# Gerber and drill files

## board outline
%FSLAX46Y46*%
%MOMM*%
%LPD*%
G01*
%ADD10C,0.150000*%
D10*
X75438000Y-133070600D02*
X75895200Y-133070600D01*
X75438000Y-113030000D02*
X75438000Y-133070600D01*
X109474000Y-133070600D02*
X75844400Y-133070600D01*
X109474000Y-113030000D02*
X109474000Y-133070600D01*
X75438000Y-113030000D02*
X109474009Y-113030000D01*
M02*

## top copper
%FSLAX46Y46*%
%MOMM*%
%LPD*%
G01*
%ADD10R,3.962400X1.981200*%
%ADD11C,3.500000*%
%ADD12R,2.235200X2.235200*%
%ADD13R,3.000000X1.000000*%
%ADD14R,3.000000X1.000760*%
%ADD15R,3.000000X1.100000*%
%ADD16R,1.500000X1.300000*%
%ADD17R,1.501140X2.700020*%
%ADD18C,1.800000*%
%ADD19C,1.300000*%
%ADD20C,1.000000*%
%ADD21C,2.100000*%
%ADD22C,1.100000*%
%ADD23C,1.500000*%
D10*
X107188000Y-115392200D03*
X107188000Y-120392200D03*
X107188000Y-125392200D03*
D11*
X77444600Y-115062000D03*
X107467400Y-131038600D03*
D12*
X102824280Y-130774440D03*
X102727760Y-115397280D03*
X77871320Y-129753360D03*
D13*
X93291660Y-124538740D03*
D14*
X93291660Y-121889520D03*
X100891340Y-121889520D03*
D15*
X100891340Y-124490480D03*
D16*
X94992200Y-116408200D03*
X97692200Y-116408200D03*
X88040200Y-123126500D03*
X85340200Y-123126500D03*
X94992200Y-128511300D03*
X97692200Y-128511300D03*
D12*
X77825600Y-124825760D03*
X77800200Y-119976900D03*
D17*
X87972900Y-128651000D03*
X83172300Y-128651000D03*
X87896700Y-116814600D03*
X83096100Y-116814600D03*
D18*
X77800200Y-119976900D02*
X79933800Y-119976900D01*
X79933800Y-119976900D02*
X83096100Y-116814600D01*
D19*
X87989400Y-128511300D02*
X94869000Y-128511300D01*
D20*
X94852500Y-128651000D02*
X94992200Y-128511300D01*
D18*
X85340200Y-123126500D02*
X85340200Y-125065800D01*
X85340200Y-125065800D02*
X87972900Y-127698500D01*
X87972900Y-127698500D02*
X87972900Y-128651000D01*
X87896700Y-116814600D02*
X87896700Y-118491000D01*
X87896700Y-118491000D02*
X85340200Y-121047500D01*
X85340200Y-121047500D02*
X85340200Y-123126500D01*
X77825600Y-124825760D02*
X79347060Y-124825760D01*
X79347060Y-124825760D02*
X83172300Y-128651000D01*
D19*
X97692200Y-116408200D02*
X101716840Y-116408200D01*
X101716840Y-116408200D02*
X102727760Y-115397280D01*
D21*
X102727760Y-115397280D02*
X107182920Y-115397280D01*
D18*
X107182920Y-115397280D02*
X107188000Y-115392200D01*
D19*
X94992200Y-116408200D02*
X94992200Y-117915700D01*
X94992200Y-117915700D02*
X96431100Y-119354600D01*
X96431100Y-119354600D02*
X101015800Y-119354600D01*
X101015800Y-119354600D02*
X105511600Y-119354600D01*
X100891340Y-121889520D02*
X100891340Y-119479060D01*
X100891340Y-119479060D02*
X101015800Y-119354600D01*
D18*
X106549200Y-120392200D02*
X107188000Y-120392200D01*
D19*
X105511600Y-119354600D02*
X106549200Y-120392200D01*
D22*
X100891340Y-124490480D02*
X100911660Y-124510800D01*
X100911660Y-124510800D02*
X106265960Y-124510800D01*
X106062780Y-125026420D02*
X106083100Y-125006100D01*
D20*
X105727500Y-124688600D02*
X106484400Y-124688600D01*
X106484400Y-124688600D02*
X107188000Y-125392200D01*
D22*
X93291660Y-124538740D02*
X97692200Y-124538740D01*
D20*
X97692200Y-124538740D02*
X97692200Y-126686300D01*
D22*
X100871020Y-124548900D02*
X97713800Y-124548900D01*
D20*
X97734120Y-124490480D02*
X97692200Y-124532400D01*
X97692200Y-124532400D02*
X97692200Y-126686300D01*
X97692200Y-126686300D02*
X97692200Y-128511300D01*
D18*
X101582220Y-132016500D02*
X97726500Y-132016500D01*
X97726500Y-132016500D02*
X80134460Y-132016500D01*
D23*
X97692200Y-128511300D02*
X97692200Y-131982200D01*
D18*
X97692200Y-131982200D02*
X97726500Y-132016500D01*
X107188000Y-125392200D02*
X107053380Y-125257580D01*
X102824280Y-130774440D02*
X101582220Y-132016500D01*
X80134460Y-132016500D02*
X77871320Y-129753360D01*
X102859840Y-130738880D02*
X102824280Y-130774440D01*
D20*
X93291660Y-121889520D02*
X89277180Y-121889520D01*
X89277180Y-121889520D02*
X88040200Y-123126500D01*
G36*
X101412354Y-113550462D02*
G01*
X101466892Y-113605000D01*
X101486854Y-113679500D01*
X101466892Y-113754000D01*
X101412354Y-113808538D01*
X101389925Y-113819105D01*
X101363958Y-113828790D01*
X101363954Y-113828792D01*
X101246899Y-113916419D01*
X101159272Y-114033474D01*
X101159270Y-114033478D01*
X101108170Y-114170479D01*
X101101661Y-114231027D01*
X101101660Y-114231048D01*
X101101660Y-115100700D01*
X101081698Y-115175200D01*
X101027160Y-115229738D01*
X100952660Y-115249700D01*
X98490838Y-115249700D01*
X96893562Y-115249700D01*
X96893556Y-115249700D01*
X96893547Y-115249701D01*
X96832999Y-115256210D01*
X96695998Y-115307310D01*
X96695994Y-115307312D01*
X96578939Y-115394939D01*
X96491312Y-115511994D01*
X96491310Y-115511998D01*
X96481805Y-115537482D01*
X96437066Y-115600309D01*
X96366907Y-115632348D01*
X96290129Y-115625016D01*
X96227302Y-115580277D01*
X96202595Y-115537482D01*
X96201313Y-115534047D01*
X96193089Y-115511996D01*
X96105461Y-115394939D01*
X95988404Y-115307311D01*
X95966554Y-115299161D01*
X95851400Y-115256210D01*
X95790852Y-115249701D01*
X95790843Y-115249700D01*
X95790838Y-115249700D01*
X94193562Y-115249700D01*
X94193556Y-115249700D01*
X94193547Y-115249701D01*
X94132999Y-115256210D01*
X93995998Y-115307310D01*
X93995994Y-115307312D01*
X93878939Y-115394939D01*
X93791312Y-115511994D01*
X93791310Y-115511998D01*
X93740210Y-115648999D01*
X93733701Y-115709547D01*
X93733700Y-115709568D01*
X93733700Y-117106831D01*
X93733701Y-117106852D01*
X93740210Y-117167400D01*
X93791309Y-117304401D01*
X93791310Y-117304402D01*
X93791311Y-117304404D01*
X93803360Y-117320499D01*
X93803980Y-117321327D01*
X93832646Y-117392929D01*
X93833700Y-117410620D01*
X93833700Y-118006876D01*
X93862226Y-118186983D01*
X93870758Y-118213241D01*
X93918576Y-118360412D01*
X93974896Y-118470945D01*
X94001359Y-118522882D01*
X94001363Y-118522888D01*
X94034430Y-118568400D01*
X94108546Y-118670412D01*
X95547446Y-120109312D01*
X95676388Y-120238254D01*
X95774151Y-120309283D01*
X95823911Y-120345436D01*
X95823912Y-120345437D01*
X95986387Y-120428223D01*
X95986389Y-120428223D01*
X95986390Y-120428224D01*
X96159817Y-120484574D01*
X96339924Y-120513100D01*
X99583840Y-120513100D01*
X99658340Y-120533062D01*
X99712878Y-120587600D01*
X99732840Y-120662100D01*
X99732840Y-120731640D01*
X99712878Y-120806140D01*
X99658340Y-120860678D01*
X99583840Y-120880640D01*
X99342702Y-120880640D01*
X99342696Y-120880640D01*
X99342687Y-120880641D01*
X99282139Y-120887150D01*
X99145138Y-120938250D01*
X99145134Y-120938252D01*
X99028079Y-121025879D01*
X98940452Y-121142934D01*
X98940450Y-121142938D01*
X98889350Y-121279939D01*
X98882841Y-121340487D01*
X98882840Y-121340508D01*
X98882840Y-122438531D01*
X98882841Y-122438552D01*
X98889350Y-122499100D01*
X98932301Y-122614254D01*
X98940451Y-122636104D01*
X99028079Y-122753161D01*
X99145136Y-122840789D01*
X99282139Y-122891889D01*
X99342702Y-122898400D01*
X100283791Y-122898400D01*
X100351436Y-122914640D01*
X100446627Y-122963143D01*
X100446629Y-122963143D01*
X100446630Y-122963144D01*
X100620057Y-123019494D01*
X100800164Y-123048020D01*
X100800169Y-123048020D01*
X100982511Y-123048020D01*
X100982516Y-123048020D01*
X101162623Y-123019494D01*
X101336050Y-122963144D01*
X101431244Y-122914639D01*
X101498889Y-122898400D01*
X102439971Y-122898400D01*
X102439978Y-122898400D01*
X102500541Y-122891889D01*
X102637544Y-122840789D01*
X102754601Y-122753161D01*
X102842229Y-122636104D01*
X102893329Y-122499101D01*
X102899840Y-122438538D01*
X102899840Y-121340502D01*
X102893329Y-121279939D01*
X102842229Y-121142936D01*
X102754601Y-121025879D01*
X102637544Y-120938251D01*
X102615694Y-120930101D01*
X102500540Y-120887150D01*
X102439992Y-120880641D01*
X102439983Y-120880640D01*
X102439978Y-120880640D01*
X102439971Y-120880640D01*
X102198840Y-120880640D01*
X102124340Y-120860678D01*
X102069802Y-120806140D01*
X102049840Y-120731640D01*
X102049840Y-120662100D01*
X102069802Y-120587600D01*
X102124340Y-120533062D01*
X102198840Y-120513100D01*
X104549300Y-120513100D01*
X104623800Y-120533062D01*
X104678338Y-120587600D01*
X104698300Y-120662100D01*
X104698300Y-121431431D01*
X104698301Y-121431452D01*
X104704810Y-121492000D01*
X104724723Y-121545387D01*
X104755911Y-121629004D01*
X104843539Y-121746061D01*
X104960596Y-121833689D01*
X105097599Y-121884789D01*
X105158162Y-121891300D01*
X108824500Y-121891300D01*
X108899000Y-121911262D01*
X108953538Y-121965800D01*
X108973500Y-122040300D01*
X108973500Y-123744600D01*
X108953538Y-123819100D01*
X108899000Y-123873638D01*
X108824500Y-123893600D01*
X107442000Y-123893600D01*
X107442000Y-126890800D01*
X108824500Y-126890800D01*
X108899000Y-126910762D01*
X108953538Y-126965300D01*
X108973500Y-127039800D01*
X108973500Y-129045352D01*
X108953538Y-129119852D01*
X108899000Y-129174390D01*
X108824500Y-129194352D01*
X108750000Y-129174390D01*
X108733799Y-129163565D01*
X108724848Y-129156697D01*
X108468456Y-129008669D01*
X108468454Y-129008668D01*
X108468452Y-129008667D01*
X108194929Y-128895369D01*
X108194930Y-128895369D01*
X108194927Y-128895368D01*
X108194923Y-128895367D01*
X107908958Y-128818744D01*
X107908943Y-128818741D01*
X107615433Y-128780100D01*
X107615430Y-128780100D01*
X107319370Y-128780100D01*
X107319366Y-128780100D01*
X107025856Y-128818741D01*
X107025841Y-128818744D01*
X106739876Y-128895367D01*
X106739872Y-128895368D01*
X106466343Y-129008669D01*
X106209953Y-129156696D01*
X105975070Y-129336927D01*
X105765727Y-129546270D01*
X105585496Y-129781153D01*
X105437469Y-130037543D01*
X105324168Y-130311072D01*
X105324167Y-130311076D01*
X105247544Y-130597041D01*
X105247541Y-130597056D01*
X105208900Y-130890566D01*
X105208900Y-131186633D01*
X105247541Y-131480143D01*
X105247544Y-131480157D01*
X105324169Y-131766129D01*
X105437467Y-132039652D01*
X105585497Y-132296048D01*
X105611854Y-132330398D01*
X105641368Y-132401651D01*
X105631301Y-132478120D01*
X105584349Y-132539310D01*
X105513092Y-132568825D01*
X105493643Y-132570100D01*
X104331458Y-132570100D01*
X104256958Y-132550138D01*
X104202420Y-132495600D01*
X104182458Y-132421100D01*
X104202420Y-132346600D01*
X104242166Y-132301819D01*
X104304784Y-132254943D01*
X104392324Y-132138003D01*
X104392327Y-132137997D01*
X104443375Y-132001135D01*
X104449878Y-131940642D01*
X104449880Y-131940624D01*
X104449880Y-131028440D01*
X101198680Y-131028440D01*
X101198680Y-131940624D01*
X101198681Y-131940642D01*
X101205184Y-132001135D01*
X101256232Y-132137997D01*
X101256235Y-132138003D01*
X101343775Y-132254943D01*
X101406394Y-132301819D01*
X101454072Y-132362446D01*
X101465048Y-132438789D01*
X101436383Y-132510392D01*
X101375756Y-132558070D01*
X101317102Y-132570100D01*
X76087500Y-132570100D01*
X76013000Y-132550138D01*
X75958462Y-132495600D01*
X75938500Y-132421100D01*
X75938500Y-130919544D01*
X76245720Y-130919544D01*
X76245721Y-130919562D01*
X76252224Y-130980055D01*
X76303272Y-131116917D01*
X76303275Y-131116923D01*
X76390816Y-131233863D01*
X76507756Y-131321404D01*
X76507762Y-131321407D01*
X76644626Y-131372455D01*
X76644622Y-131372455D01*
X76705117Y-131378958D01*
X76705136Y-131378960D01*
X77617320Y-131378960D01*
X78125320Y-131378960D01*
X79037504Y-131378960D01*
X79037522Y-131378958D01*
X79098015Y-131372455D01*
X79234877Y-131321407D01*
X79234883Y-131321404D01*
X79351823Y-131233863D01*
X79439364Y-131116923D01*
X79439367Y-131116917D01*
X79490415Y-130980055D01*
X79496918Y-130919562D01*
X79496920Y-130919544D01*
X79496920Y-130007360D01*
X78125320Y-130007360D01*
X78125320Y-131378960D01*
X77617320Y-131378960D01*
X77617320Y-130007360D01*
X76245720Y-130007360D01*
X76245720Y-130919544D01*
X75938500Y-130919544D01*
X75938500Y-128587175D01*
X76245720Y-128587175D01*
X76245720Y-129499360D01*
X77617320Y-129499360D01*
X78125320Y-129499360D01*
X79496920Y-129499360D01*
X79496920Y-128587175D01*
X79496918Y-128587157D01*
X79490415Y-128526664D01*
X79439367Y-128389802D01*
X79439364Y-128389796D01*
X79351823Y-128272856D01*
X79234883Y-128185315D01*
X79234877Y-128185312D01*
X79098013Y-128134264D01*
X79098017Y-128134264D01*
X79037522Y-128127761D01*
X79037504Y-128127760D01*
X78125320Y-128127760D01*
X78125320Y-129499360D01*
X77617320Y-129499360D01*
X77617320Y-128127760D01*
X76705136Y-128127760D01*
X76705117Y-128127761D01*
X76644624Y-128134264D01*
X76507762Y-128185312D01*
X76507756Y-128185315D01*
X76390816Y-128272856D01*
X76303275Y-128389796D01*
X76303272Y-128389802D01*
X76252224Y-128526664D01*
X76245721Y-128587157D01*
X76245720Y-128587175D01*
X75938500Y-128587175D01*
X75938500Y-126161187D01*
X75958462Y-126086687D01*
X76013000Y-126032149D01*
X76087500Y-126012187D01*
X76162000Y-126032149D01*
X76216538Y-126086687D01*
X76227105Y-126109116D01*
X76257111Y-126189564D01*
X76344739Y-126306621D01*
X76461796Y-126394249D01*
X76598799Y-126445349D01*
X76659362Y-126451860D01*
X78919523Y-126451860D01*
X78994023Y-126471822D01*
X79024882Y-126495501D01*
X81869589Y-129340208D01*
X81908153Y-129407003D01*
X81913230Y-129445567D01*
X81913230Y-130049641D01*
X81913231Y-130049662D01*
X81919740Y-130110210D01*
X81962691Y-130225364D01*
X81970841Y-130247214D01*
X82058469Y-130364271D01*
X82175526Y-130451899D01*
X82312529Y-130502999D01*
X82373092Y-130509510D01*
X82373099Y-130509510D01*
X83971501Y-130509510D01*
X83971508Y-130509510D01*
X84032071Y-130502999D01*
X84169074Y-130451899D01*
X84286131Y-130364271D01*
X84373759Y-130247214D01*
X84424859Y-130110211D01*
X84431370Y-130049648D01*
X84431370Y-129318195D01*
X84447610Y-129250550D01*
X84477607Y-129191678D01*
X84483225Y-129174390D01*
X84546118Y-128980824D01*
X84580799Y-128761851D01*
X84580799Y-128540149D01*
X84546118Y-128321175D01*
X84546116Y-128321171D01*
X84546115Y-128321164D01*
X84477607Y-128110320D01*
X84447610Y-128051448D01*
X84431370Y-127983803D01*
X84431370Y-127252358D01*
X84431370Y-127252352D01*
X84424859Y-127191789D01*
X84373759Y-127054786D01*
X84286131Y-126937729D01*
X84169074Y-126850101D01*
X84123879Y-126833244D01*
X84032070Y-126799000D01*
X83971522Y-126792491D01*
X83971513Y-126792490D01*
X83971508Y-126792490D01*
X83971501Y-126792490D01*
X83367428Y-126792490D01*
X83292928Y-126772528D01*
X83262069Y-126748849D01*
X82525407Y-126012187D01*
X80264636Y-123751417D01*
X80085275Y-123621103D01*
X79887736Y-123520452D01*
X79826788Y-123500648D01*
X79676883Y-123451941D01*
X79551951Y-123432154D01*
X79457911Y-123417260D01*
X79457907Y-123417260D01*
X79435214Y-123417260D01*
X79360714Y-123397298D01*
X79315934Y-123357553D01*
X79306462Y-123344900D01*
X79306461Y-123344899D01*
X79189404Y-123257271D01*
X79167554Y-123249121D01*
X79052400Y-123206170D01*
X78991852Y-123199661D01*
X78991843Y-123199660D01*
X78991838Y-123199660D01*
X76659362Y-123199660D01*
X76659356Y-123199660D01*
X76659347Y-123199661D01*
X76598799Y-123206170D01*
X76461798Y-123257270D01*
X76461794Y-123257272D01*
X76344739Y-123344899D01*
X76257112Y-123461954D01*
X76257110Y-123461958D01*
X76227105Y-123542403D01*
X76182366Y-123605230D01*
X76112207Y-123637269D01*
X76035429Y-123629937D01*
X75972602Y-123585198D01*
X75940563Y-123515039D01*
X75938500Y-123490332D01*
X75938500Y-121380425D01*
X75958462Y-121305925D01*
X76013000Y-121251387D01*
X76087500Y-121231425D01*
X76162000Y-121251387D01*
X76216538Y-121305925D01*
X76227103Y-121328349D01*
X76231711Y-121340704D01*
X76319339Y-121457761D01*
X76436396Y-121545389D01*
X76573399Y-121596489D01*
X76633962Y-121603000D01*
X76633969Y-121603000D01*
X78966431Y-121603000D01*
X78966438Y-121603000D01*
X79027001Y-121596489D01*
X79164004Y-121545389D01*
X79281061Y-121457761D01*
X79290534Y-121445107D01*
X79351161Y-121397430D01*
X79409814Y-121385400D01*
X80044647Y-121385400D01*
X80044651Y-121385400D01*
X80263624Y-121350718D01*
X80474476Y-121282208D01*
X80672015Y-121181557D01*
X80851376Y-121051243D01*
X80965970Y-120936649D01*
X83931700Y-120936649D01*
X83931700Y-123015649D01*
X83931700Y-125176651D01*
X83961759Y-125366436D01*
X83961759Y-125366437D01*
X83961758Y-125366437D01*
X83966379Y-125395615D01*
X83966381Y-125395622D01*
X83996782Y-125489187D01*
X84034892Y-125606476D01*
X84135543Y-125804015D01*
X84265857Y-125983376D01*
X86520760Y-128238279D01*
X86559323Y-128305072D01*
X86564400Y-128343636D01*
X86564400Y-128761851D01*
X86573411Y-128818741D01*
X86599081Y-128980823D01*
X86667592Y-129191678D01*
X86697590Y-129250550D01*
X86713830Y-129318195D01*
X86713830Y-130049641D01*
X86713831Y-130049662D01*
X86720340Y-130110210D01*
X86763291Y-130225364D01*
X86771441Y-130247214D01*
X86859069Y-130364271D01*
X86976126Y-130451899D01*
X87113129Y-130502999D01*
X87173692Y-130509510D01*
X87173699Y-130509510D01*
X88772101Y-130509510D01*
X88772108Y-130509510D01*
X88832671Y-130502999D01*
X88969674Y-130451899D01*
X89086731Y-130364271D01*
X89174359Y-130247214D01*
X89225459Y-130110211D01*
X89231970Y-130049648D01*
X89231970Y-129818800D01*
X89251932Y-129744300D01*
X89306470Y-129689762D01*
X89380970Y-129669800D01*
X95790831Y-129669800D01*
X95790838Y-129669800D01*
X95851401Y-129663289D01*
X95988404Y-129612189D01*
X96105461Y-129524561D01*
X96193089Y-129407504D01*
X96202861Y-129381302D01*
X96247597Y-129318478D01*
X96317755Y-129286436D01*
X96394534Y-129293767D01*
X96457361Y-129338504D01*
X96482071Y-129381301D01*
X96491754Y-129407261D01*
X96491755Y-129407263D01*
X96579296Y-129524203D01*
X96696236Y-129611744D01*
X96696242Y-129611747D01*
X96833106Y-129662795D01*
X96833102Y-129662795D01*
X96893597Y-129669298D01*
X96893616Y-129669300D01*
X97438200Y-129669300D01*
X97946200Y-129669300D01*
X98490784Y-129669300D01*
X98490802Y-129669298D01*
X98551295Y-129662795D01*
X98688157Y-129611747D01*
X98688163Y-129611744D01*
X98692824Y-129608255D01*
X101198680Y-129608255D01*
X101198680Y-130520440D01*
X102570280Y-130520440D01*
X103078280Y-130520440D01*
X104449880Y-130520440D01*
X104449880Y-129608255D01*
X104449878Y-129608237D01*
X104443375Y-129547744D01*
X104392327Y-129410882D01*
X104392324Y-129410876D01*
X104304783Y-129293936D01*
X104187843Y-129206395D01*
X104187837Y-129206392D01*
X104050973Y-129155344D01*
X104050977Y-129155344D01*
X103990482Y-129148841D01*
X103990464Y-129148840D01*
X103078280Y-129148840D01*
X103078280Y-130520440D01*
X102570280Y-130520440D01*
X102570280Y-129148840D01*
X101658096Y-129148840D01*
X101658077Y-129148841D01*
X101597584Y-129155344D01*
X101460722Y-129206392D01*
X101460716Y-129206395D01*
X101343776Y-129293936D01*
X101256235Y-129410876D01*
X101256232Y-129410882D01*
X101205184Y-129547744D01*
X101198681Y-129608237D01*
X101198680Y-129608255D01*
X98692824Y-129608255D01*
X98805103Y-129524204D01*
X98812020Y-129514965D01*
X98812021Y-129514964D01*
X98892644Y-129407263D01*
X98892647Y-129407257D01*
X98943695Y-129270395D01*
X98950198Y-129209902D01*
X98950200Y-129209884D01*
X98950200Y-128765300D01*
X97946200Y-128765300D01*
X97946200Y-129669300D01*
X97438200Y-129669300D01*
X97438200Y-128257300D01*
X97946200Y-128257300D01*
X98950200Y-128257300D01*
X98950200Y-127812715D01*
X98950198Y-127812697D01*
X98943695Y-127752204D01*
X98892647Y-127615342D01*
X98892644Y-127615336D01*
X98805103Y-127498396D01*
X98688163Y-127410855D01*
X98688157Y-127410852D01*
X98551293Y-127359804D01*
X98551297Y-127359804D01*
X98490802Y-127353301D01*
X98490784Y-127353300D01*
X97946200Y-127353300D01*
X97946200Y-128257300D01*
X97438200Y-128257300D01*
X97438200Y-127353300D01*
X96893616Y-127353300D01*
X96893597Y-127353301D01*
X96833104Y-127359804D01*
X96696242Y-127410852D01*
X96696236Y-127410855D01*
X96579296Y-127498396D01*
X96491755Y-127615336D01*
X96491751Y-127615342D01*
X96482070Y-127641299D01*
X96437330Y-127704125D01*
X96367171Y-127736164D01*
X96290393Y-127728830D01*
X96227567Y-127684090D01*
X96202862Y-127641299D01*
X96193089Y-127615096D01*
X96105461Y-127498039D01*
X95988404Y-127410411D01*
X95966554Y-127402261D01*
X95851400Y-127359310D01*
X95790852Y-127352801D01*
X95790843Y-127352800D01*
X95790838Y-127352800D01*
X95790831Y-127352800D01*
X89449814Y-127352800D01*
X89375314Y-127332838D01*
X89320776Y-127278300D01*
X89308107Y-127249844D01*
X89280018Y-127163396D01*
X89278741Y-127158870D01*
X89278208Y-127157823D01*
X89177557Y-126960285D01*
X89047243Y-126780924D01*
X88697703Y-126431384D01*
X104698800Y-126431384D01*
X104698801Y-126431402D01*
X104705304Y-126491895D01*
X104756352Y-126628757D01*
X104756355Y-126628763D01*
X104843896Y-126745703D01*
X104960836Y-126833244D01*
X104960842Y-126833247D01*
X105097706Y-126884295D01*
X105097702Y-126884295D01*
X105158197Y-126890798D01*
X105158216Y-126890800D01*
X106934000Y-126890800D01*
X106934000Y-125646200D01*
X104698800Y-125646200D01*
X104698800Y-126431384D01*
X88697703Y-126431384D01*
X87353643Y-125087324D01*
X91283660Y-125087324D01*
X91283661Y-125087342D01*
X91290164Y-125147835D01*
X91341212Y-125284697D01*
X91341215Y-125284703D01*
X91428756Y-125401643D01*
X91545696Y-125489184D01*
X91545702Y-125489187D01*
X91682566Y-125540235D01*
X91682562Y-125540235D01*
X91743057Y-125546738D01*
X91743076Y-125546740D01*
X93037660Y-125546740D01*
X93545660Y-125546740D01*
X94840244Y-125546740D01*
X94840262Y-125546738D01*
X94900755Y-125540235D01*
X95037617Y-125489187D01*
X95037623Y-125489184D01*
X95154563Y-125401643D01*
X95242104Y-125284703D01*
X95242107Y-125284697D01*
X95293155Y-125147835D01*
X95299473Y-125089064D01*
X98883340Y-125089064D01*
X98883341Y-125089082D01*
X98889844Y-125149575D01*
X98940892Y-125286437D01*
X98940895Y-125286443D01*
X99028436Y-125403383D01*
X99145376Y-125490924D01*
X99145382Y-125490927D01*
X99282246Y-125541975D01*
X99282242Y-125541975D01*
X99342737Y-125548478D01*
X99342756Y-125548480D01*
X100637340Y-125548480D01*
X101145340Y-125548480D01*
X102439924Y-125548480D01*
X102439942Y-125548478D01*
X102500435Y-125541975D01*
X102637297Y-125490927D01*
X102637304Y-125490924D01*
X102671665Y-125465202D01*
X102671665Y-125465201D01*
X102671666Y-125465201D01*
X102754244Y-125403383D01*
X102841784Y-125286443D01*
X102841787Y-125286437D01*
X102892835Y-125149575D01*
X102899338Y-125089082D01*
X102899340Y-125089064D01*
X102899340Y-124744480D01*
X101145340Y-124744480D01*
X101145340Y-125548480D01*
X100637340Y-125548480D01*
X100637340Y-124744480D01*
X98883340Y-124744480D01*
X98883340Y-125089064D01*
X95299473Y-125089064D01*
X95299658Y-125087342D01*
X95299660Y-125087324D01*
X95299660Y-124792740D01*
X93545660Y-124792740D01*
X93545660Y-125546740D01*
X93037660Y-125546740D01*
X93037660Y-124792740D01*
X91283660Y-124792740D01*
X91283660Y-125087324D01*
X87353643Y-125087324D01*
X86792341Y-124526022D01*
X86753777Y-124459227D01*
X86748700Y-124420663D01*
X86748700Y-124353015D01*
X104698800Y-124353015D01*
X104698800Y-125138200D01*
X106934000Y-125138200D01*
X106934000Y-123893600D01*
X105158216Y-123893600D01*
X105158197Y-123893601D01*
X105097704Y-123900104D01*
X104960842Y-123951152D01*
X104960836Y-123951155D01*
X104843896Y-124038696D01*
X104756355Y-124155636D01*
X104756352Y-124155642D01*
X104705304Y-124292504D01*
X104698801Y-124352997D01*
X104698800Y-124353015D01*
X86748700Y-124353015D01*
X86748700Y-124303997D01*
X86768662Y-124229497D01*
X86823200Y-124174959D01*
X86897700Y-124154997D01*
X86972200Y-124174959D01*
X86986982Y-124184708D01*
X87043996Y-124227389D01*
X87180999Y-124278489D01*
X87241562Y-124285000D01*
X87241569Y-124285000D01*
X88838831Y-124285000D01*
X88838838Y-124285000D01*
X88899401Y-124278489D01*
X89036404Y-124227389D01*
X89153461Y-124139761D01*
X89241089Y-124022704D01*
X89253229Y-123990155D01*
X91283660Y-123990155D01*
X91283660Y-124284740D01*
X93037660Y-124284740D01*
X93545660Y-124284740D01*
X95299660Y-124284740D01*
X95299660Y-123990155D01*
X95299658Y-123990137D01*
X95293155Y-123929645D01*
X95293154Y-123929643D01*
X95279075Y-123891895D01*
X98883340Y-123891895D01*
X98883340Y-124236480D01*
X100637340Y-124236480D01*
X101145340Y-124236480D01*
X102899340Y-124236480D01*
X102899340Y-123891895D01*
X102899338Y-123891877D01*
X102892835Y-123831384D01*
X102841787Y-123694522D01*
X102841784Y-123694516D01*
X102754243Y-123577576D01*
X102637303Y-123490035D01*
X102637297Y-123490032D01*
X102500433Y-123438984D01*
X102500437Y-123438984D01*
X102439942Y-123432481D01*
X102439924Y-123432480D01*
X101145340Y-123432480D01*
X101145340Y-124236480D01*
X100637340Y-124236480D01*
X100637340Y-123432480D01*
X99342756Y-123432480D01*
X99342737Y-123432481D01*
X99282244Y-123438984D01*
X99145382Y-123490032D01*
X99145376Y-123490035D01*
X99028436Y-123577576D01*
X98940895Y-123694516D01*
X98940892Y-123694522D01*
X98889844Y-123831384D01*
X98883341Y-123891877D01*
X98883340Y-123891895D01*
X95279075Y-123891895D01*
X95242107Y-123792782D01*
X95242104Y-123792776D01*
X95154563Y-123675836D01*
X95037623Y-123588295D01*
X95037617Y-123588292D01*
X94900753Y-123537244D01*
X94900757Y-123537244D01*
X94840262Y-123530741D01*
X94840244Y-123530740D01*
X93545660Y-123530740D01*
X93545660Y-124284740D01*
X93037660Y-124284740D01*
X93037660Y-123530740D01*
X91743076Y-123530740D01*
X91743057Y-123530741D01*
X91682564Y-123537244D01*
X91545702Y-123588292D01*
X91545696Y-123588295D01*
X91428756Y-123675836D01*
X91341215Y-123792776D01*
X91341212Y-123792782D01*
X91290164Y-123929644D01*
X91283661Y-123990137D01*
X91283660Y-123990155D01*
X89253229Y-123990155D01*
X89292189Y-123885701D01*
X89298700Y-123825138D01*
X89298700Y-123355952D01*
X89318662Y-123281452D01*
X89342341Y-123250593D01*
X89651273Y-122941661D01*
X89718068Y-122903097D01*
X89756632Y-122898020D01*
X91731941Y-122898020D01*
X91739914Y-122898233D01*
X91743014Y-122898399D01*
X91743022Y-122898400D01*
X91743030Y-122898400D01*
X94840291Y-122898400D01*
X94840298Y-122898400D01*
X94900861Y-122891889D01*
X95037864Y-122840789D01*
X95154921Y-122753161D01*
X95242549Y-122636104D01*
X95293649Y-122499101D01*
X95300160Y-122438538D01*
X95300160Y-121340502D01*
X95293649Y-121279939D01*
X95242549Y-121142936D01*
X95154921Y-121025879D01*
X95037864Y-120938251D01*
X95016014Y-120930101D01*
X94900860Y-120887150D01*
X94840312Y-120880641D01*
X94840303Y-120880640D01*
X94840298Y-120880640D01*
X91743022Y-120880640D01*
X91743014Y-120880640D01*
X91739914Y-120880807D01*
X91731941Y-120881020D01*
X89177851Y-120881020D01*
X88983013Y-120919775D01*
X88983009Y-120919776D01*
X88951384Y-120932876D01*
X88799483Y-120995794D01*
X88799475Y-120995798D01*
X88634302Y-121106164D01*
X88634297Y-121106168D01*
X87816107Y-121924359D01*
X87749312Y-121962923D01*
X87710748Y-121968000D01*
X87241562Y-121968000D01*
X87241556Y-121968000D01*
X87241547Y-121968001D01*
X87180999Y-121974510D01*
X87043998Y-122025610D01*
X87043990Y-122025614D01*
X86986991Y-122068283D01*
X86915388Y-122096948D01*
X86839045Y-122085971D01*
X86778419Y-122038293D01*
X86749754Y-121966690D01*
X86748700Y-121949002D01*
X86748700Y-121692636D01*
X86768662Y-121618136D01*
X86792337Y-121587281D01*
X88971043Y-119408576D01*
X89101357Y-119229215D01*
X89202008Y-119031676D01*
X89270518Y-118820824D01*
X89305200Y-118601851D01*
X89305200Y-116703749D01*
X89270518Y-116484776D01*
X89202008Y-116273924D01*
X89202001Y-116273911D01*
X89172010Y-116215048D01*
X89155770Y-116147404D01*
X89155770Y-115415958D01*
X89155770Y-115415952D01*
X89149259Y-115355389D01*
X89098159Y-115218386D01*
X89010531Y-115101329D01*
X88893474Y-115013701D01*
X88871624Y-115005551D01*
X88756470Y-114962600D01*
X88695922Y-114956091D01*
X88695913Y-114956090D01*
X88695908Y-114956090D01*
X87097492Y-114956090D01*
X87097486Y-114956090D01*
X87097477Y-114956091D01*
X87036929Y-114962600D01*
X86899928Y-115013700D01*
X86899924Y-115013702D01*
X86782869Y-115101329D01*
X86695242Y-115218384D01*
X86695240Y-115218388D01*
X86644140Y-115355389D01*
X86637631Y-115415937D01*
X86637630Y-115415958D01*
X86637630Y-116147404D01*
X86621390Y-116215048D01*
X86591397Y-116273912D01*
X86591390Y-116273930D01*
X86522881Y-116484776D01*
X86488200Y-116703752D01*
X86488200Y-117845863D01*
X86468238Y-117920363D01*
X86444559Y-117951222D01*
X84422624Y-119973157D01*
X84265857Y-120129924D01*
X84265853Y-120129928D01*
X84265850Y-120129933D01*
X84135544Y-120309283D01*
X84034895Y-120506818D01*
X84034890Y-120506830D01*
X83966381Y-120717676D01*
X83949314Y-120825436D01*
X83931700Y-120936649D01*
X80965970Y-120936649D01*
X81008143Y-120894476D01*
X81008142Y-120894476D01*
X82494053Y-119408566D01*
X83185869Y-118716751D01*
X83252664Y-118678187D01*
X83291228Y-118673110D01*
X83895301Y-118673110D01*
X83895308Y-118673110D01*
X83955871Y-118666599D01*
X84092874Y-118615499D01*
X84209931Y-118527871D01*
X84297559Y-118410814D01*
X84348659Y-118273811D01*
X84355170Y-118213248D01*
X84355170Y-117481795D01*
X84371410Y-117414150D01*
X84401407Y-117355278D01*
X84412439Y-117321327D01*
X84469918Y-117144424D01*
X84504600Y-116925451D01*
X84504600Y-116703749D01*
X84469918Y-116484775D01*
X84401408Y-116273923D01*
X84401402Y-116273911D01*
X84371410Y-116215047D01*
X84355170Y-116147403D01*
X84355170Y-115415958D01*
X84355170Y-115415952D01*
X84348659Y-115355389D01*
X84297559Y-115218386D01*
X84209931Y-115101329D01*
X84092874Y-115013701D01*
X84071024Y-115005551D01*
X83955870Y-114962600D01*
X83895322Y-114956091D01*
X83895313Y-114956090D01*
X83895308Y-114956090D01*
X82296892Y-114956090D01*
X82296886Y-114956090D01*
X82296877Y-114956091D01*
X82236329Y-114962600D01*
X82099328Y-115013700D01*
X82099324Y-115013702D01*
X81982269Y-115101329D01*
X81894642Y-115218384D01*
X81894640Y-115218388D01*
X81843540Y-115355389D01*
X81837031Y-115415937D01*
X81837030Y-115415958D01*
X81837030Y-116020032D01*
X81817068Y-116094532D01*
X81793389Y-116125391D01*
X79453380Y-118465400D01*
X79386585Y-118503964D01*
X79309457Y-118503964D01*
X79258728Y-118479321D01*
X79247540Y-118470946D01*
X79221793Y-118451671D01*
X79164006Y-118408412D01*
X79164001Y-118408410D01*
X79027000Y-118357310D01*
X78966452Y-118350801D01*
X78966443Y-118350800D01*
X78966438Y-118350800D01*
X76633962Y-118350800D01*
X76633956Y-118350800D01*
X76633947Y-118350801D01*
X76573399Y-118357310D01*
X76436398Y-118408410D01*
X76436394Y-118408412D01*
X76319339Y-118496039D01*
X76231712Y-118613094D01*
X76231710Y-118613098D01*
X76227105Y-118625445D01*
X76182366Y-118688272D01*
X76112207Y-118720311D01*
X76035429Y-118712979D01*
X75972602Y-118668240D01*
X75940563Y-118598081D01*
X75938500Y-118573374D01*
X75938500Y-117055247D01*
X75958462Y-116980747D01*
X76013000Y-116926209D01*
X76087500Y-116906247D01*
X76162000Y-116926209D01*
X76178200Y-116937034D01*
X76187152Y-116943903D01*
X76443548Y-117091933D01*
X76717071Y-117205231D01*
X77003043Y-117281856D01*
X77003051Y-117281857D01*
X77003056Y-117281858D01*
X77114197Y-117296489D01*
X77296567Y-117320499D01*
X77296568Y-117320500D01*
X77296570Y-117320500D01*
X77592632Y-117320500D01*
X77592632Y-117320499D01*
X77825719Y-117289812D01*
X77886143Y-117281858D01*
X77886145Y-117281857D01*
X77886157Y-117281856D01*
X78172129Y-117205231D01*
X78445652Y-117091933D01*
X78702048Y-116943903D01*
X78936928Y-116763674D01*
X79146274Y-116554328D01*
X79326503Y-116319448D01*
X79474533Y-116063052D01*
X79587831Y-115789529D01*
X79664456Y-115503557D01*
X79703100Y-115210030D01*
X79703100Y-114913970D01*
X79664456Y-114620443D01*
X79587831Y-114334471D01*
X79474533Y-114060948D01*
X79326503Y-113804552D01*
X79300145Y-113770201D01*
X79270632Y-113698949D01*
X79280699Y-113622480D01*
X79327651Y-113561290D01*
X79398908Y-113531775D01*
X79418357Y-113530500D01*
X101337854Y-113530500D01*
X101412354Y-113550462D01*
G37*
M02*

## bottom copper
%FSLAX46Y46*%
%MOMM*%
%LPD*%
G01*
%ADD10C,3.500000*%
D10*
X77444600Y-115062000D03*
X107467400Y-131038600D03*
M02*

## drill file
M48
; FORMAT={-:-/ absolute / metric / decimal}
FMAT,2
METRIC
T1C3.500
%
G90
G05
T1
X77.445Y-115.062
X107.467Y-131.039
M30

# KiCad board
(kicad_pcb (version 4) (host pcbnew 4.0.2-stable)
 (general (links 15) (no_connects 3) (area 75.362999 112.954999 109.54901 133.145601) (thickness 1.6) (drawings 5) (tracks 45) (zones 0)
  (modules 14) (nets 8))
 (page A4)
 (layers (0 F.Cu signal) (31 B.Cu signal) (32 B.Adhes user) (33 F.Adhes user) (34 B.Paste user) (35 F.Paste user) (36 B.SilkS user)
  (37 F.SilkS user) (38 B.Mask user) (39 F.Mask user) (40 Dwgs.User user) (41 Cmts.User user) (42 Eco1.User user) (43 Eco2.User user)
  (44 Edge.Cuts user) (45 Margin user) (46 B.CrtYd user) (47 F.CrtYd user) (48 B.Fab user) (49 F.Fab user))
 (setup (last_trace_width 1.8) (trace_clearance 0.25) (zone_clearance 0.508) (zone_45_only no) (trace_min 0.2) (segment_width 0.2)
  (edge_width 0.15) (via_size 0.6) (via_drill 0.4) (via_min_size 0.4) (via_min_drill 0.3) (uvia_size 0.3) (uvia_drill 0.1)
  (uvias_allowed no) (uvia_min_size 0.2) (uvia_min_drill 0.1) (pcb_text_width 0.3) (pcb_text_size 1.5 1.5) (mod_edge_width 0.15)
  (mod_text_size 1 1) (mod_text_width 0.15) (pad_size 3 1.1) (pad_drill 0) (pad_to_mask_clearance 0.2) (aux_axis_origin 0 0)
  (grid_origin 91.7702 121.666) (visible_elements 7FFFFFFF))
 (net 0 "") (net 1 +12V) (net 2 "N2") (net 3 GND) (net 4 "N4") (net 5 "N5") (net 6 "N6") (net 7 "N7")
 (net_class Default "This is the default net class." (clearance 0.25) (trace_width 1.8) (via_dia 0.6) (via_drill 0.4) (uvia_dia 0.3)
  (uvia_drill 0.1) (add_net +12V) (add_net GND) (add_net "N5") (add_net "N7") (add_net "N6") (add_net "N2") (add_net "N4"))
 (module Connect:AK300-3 (layer F.Cu) (at 107.188 115.3922 270)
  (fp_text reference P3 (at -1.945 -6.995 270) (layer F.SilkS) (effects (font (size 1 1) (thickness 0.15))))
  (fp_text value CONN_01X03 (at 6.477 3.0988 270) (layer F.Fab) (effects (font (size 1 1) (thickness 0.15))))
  (pad 1 smd rect (at 0 0 270) (size 1.9812 3.9624) (layers F.Cu F.Paste F.Mask) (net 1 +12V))
  (pad 2 smd rect (at 5 0 270) (size 1.9812 3.9624) (layers F.Cu F.Paste F.Mask) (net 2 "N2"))
  (pad 3 smd rect (at 10 0 270) (size 1.9812 3.9624) (layers F.Cu F.Paste F.Mask) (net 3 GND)))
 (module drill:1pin (layer F.Cu) (at 77.4446 115.062)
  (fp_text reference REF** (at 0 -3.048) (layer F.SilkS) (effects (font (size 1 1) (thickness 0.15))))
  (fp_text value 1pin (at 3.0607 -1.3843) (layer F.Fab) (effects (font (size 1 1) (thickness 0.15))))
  (pad 1 thru_hole circle (at 0 0) (size 3.5 3.5) (drill 3.5) (layers *.Cu *.Mask F.SilkS)))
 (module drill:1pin (layer F.Cu) (at 107.4674 131.0386)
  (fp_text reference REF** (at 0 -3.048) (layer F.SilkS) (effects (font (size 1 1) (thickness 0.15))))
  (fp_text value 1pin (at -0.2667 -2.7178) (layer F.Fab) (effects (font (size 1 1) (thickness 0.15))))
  (pad 1 thru_hole circle (at 0 0) (size 3.5 3.5) (drill 3.5) (layers *.Cu *.Mask F.SilkS)))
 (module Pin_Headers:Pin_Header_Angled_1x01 (layer F.Cu) (at 102.82428 130.77444 270)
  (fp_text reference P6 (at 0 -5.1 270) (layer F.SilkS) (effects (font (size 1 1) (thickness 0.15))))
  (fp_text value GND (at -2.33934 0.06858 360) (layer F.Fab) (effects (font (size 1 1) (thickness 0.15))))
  (pad 1 smd rect (at 0 0 270) (size 2.2352 2.2352) (layers F.Cu F.Paste F.Mask) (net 3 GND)))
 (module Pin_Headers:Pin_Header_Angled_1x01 (layer F.Cu) (at 102.72776 115.39728 90)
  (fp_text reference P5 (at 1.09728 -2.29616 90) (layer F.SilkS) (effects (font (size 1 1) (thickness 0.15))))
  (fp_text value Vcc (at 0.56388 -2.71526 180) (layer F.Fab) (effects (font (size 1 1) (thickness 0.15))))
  (pad 1 smd rect (at 0 0 90) (size 2.2352 2.2352) (layers F.Cu F.Paste F.Mask) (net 1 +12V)))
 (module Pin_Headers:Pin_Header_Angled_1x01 (layer F.Cu) (at 77.87132 129.75336 180)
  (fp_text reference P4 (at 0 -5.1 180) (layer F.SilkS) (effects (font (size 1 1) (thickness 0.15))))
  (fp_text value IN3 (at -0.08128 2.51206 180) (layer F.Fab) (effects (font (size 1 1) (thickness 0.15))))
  (pad 1 smd rect (at 0 0 180) (size 2.2352 2.2352) (layers F.Cu F.Paste F.Mask) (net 3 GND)))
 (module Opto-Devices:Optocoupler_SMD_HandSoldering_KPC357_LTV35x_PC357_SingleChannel (layer F.Cu) (at 97.0915 123.19)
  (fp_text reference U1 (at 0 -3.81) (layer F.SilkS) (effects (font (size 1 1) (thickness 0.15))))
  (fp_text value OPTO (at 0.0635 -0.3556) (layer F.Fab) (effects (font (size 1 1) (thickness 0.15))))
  (pad 2 smd rect (at -3.79984 1.34874) (size 3 1) (layers F.Cu F.Paste F.Mask) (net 3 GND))
  (pad 1 smd rect (at -3.79984 -1.30048) (size 3 1.00076) (layers F.Cu F.Paste F.Mask) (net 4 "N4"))
  (pad 4 smd rect (at 3.79984 -1.30048) (size 3 1.00076) (layers F.Cu F.Paste F.Mask) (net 2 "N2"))
  (pad 3 smd rect (at 3.79984 1.30048) (size 3 1.1) (layers F.Cu F.Paste F.Mask) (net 3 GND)))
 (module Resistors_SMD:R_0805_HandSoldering (layer F.Cu) (at 96.3422 116.4082)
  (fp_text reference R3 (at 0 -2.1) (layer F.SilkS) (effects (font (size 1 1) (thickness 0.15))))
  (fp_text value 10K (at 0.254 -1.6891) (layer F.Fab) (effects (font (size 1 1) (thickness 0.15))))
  (pad 1 smd rect (at -1.35 0) (size 1.5 1.3) (layers F.Cu F.Paste F.Mask) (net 2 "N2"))
  (pad 2 smd rect (at 1.35 0) (size 1.5 1.3) (layers F.Cu F.Paste F.Mask) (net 1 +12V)))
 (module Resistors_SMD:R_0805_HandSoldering (layer F.Cu) (at 86.6902 123.1265 180)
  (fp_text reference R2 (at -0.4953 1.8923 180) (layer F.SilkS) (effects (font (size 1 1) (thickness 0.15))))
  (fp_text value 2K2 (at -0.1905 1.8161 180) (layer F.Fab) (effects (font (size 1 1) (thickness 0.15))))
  (pad 1 smd rect (at -1.35 0 180) (size 1.5 1.3) (layers F.Cu F.Paste F.Mask) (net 4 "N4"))
  (pad 2 smd rect (at 1.35 0 180) (size 1.5 1.3) (layers F.Cu F.Paste F.Mask) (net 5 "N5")))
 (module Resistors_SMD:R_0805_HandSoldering (layer F.Cu) (at 96.3422 128.5113)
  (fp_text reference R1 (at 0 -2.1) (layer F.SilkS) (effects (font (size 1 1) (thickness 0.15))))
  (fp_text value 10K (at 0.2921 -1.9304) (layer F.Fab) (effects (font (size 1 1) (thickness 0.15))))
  (pad 1 smd rect (at -1.35 0) (size 1.5 1.3) (layers F.Cu F.Paste F.Mask) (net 5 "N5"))
  (pad 2 smd rect (at 1.35 0) (size 1.5 1.3) (layers F.Cu F.Paste F.Mask) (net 3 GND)))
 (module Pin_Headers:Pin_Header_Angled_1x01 (layer F.Cu) (at 77.8256 124.82576 180)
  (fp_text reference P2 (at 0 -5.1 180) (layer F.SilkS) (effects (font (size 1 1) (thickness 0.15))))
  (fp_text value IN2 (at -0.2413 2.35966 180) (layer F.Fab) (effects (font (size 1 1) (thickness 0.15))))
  (pad 1 smd rect (at 0 0 180) (size 2.2352 2.2352) (layers F.Cu F.Paste F.Mask) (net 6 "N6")))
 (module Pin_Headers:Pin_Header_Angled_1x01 (layer F.Cu) (at 77.8002 119.9769 180)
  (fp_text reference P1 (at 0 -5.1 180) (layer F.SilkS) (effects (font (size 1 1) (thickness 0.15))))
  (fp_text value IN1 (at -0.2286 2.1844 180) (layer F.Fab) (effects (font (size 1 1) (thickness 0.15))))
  (pad 1 smd rect (at 0 0 180) (size 2.2352 2.2352) (layers F.Cu F.Paste F.Mask) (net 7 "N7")))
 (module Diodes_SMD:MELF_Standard (layer F.Cu) (at 85.5726 128.651 180)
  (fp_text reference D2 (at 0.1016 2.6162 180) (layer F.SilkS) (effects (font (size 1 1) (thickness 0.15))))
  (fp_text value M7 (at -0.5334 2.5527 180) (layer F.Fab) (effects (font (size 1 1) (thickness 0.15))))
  (pad 1 smd rect (at -2.4003 0 180) (size 1.50114 2.70002) (layers F.Cu F.Paste F.Mask) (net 5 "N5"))
  (pad 2 smd rect (at 2.4003 0 180) (size 1.50114 2.70002) (layers F.Cu F.Paste F.Mask) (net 6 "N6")))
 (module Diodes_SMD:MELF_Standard (layer F.Cu) (at 85.4964 116.8146 180)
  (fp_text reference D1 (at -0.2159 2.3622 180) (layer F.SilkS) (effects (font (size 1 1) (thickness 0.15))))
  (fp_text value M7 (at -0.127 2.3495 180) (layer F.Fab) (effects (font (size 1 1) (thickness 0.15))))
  (pad 1 smd rect (at -2.4003 0 180) (size 1.50114 2.70002) (layers F.Cu F.Paste F.Mask) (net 5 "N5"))
  (pad 2 smd rect (at 2.4003 0 180) (size 1.50114 2.70002) (layers F.Cu F.Paste F.Mask) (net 7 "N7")))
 (gr_line (start 75.438 133.0706) (end 75.8952 133.0706) (layer Edge.Cuts) (width 0.15))
 (gr_line (start 75.438 113.03) (end 75.438 133.0706) (layer Edge.Cuts) (width 0.15))
 (gr_line (start 109.474 133.0706) (end 75.8444 133.0706) (layer Edge.Cuts) (width 0.15))
 (gr_line (start 109.474 113.03) (end 109.474 133.0706) (layer Edge.Cuts) (width 0.15))
 (gr_line (start 75.438 113.03) (end 109.474009 113.03) (layer Edge.Cuts) (width 0.15))
 (segment (start 77.8002 119.9769) (end 79.9338 119.9769) (width 1.8) (layer F.Cu) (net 7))
 (segment (start 79.9338 119.9769) (end 83.0961 116.8146) (width 1.8) (layer F.Cu) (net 7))
 (segment (start 87.9894 128.5113) (end 94.869 128.5113) (width 1.3) (layer F.Cu) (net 5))
 (segment (start 94.8525 128.651) (end 94.9922 128.5113) (width 1) (layer F.Cu) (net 5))
 (segment (start 85.3402 123.1265) (end 85.3402 125.0658) (width 1.8) (layer F.Cu) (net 5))
 (segment (start 85.3402 125.0658) (end 87.9729 127.6985) (width 1.8) (layer F.Cu) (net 5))
 (segment (start 87.9729 127.6985) (end 87.9729 128.651) (width 1.8) (layer F.Cu) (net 5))
 (segment (start 87.8967 116.8146) (end 87.8967 118.491) (width 1.8) (layer F.Cu) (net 5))
 (segment (start 87.8967 118.491) (end 85.3402 121.0475) (width 1.8) (layer F.Cu) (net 5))
 (segment (start 85.3402 121.0475) (end 85.3402 123.1265) (width 1.8) (layer F.Cu) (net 5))
 (segment (start 77.8256 124.82576) (end 79.34706 124.82576) (width 1.8) (layer F.Cu) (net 6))
 (segment (start 79.34706 124.82576) (end 83.1723 128.651) (width 1.8) (layer F.Cu) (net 6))
 (segment (start 97.6922 116.4082) (end 101.71684 116.4082) (width 1.3) (layer F.Cu) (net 1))
 (segment (start 101.71684 116.4082) (end 102.72776 115.39728) (width 1.3) (layer F.Cu) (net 1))
 (segment (start 102.72776 115.39728) (end 107.18292 115.39728) (width 2.1) (layer F.Cu) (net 1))
 (segment (start 107.18292 115.39728) (end 107.188 115.3922) (width 1.8) (layer F.Cu) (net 1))
 (segment (start 94.9922 116.4082) (end 94.9922 117.9157) (width 1.3) (layer F.Cu) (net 2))
 (segment (start 94.9922 117.9157) (end 96.4311 119.3546) (width 1.3) (layer F.Cu) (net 2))
 (segment (start 96.4311 119.3546) (end 101.0158 119.3546) (width 1.3) (layer F.Cu) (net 2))
 (segment (start 101.0158 119.3546) (end 105.5116 119.3546) (width 1.3) (layer F.Cu) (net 2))
 (segment (start 100.89134 121.88952) (end 100.89134 119.47906) (width 1.3) (layer F.Cu) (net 2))
 (segment (start 100.89134 119.47906) (end 101.0158 119.3546) (width 1.3) (layer F.Cu) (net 2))
 (segment (start 106.5492 120.3922) (end 107.188 120.3922) (width 1.8) (layer F.Cu) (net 2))
 (segment (start 105.5116 119.3546) (end 106.5492 120.3922) (width 1.3) (layer F.Cu) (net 2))
 (segment (start 100.89134 124.49048) (end 100.91166 124.5108) (width 1.1) (layer F.Cu) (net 3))
 (segment (start 100.91166 124.5108) (end 106.26596 124.5108) (width 1.1) (layer F.Cu) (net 3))
 (segment (start 106.06278 125.02642) (end 106.0831 125.0061) (width 1.1) (layer F.Cu) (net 3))
 (segment (start 105.7275 124.6886) (end 106.4844 124.6886) (width 1) (layer F.Cu) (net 3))
 (segment (start 106.4844 124.6886) (end 107.188 125.3922) (width 1) (layer F.Cu) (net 3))
 (segment (start 93.29166 124.53874) (end 97.6922 124.53874) (width 1.1) (layer F.Cu) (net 3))
 (segment (start 97.6922 124.53874) (end 97.6922 126.6863) (width 1) (layer F.Cu) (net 3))
 (segment (start 100.87102 124.5489) (end 97.7138 124.5489) (width 1.1) (layer F.Cu) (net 3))
 (segment (start 97.73412 124.49048) (end 97.6922 124.5324) (width 1) (layer F.Cu) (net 3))
 (segment (start 97.6922 124.5324) (end 97.6922 126.6863) (width 1) (layer F.Cu) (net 3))
 (segment (start 97.6922 126.6863) (end 97.6922 128.5113) (width 1) (layer F.Cu) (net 3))
 (segment (start 101.58222 132.0165) (end 97.7265 132.0165) (width 1.8) (layer F.Cu) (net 3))
 (segment (start 97.7265 132.0165) (end 80.13446 132.0165) (width 1.8) (layer F.Cu) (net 3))
 (segment (start 97.6922 128.5113) (end 97.6922 131.9822) (width 1.5) (layer F.Cu) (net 3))
 (segment (start 97.6922 131.9822) (end 97.7265 132.0165) (width 1.8) (layer F.Cu) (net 3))
 (segment (start 107.188 125.3922) (end 107.05338 125.25758) (width 1.8) (layer F.Cu) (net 3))
 (segment (start 102.82428 130.77444) (end 101.58222 132.0165) (width 1.8) (layer F.Cu) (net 3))
 (segment (start 80.13446 132.0165) (end 77.87132 129.75336) (width 1.8) (layer F.Cu) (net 3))
 (segment (start 102.85984 130.73888) (end 102.82428 130.77444) (width 1.8) (layer F.Cu) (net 3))
 (segment (start 93.29166 121.88952) (end 89.27718 121.88952) (width 1) (layer F.Cu) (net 4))
 (segment (start 89.27718 121.88952) (end 88.0402 123.1265) (width 1) (layer F.Cu) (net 4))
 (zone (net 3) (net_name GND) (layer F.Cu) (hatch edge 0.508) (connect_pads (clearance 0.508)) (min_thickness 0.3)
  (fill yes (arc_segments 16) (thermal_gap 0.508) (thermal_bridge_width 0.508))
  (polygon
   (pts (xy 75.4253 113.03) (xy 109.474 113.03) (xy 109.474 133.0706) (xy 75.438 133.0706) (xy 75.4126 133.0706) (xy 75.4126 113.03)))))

